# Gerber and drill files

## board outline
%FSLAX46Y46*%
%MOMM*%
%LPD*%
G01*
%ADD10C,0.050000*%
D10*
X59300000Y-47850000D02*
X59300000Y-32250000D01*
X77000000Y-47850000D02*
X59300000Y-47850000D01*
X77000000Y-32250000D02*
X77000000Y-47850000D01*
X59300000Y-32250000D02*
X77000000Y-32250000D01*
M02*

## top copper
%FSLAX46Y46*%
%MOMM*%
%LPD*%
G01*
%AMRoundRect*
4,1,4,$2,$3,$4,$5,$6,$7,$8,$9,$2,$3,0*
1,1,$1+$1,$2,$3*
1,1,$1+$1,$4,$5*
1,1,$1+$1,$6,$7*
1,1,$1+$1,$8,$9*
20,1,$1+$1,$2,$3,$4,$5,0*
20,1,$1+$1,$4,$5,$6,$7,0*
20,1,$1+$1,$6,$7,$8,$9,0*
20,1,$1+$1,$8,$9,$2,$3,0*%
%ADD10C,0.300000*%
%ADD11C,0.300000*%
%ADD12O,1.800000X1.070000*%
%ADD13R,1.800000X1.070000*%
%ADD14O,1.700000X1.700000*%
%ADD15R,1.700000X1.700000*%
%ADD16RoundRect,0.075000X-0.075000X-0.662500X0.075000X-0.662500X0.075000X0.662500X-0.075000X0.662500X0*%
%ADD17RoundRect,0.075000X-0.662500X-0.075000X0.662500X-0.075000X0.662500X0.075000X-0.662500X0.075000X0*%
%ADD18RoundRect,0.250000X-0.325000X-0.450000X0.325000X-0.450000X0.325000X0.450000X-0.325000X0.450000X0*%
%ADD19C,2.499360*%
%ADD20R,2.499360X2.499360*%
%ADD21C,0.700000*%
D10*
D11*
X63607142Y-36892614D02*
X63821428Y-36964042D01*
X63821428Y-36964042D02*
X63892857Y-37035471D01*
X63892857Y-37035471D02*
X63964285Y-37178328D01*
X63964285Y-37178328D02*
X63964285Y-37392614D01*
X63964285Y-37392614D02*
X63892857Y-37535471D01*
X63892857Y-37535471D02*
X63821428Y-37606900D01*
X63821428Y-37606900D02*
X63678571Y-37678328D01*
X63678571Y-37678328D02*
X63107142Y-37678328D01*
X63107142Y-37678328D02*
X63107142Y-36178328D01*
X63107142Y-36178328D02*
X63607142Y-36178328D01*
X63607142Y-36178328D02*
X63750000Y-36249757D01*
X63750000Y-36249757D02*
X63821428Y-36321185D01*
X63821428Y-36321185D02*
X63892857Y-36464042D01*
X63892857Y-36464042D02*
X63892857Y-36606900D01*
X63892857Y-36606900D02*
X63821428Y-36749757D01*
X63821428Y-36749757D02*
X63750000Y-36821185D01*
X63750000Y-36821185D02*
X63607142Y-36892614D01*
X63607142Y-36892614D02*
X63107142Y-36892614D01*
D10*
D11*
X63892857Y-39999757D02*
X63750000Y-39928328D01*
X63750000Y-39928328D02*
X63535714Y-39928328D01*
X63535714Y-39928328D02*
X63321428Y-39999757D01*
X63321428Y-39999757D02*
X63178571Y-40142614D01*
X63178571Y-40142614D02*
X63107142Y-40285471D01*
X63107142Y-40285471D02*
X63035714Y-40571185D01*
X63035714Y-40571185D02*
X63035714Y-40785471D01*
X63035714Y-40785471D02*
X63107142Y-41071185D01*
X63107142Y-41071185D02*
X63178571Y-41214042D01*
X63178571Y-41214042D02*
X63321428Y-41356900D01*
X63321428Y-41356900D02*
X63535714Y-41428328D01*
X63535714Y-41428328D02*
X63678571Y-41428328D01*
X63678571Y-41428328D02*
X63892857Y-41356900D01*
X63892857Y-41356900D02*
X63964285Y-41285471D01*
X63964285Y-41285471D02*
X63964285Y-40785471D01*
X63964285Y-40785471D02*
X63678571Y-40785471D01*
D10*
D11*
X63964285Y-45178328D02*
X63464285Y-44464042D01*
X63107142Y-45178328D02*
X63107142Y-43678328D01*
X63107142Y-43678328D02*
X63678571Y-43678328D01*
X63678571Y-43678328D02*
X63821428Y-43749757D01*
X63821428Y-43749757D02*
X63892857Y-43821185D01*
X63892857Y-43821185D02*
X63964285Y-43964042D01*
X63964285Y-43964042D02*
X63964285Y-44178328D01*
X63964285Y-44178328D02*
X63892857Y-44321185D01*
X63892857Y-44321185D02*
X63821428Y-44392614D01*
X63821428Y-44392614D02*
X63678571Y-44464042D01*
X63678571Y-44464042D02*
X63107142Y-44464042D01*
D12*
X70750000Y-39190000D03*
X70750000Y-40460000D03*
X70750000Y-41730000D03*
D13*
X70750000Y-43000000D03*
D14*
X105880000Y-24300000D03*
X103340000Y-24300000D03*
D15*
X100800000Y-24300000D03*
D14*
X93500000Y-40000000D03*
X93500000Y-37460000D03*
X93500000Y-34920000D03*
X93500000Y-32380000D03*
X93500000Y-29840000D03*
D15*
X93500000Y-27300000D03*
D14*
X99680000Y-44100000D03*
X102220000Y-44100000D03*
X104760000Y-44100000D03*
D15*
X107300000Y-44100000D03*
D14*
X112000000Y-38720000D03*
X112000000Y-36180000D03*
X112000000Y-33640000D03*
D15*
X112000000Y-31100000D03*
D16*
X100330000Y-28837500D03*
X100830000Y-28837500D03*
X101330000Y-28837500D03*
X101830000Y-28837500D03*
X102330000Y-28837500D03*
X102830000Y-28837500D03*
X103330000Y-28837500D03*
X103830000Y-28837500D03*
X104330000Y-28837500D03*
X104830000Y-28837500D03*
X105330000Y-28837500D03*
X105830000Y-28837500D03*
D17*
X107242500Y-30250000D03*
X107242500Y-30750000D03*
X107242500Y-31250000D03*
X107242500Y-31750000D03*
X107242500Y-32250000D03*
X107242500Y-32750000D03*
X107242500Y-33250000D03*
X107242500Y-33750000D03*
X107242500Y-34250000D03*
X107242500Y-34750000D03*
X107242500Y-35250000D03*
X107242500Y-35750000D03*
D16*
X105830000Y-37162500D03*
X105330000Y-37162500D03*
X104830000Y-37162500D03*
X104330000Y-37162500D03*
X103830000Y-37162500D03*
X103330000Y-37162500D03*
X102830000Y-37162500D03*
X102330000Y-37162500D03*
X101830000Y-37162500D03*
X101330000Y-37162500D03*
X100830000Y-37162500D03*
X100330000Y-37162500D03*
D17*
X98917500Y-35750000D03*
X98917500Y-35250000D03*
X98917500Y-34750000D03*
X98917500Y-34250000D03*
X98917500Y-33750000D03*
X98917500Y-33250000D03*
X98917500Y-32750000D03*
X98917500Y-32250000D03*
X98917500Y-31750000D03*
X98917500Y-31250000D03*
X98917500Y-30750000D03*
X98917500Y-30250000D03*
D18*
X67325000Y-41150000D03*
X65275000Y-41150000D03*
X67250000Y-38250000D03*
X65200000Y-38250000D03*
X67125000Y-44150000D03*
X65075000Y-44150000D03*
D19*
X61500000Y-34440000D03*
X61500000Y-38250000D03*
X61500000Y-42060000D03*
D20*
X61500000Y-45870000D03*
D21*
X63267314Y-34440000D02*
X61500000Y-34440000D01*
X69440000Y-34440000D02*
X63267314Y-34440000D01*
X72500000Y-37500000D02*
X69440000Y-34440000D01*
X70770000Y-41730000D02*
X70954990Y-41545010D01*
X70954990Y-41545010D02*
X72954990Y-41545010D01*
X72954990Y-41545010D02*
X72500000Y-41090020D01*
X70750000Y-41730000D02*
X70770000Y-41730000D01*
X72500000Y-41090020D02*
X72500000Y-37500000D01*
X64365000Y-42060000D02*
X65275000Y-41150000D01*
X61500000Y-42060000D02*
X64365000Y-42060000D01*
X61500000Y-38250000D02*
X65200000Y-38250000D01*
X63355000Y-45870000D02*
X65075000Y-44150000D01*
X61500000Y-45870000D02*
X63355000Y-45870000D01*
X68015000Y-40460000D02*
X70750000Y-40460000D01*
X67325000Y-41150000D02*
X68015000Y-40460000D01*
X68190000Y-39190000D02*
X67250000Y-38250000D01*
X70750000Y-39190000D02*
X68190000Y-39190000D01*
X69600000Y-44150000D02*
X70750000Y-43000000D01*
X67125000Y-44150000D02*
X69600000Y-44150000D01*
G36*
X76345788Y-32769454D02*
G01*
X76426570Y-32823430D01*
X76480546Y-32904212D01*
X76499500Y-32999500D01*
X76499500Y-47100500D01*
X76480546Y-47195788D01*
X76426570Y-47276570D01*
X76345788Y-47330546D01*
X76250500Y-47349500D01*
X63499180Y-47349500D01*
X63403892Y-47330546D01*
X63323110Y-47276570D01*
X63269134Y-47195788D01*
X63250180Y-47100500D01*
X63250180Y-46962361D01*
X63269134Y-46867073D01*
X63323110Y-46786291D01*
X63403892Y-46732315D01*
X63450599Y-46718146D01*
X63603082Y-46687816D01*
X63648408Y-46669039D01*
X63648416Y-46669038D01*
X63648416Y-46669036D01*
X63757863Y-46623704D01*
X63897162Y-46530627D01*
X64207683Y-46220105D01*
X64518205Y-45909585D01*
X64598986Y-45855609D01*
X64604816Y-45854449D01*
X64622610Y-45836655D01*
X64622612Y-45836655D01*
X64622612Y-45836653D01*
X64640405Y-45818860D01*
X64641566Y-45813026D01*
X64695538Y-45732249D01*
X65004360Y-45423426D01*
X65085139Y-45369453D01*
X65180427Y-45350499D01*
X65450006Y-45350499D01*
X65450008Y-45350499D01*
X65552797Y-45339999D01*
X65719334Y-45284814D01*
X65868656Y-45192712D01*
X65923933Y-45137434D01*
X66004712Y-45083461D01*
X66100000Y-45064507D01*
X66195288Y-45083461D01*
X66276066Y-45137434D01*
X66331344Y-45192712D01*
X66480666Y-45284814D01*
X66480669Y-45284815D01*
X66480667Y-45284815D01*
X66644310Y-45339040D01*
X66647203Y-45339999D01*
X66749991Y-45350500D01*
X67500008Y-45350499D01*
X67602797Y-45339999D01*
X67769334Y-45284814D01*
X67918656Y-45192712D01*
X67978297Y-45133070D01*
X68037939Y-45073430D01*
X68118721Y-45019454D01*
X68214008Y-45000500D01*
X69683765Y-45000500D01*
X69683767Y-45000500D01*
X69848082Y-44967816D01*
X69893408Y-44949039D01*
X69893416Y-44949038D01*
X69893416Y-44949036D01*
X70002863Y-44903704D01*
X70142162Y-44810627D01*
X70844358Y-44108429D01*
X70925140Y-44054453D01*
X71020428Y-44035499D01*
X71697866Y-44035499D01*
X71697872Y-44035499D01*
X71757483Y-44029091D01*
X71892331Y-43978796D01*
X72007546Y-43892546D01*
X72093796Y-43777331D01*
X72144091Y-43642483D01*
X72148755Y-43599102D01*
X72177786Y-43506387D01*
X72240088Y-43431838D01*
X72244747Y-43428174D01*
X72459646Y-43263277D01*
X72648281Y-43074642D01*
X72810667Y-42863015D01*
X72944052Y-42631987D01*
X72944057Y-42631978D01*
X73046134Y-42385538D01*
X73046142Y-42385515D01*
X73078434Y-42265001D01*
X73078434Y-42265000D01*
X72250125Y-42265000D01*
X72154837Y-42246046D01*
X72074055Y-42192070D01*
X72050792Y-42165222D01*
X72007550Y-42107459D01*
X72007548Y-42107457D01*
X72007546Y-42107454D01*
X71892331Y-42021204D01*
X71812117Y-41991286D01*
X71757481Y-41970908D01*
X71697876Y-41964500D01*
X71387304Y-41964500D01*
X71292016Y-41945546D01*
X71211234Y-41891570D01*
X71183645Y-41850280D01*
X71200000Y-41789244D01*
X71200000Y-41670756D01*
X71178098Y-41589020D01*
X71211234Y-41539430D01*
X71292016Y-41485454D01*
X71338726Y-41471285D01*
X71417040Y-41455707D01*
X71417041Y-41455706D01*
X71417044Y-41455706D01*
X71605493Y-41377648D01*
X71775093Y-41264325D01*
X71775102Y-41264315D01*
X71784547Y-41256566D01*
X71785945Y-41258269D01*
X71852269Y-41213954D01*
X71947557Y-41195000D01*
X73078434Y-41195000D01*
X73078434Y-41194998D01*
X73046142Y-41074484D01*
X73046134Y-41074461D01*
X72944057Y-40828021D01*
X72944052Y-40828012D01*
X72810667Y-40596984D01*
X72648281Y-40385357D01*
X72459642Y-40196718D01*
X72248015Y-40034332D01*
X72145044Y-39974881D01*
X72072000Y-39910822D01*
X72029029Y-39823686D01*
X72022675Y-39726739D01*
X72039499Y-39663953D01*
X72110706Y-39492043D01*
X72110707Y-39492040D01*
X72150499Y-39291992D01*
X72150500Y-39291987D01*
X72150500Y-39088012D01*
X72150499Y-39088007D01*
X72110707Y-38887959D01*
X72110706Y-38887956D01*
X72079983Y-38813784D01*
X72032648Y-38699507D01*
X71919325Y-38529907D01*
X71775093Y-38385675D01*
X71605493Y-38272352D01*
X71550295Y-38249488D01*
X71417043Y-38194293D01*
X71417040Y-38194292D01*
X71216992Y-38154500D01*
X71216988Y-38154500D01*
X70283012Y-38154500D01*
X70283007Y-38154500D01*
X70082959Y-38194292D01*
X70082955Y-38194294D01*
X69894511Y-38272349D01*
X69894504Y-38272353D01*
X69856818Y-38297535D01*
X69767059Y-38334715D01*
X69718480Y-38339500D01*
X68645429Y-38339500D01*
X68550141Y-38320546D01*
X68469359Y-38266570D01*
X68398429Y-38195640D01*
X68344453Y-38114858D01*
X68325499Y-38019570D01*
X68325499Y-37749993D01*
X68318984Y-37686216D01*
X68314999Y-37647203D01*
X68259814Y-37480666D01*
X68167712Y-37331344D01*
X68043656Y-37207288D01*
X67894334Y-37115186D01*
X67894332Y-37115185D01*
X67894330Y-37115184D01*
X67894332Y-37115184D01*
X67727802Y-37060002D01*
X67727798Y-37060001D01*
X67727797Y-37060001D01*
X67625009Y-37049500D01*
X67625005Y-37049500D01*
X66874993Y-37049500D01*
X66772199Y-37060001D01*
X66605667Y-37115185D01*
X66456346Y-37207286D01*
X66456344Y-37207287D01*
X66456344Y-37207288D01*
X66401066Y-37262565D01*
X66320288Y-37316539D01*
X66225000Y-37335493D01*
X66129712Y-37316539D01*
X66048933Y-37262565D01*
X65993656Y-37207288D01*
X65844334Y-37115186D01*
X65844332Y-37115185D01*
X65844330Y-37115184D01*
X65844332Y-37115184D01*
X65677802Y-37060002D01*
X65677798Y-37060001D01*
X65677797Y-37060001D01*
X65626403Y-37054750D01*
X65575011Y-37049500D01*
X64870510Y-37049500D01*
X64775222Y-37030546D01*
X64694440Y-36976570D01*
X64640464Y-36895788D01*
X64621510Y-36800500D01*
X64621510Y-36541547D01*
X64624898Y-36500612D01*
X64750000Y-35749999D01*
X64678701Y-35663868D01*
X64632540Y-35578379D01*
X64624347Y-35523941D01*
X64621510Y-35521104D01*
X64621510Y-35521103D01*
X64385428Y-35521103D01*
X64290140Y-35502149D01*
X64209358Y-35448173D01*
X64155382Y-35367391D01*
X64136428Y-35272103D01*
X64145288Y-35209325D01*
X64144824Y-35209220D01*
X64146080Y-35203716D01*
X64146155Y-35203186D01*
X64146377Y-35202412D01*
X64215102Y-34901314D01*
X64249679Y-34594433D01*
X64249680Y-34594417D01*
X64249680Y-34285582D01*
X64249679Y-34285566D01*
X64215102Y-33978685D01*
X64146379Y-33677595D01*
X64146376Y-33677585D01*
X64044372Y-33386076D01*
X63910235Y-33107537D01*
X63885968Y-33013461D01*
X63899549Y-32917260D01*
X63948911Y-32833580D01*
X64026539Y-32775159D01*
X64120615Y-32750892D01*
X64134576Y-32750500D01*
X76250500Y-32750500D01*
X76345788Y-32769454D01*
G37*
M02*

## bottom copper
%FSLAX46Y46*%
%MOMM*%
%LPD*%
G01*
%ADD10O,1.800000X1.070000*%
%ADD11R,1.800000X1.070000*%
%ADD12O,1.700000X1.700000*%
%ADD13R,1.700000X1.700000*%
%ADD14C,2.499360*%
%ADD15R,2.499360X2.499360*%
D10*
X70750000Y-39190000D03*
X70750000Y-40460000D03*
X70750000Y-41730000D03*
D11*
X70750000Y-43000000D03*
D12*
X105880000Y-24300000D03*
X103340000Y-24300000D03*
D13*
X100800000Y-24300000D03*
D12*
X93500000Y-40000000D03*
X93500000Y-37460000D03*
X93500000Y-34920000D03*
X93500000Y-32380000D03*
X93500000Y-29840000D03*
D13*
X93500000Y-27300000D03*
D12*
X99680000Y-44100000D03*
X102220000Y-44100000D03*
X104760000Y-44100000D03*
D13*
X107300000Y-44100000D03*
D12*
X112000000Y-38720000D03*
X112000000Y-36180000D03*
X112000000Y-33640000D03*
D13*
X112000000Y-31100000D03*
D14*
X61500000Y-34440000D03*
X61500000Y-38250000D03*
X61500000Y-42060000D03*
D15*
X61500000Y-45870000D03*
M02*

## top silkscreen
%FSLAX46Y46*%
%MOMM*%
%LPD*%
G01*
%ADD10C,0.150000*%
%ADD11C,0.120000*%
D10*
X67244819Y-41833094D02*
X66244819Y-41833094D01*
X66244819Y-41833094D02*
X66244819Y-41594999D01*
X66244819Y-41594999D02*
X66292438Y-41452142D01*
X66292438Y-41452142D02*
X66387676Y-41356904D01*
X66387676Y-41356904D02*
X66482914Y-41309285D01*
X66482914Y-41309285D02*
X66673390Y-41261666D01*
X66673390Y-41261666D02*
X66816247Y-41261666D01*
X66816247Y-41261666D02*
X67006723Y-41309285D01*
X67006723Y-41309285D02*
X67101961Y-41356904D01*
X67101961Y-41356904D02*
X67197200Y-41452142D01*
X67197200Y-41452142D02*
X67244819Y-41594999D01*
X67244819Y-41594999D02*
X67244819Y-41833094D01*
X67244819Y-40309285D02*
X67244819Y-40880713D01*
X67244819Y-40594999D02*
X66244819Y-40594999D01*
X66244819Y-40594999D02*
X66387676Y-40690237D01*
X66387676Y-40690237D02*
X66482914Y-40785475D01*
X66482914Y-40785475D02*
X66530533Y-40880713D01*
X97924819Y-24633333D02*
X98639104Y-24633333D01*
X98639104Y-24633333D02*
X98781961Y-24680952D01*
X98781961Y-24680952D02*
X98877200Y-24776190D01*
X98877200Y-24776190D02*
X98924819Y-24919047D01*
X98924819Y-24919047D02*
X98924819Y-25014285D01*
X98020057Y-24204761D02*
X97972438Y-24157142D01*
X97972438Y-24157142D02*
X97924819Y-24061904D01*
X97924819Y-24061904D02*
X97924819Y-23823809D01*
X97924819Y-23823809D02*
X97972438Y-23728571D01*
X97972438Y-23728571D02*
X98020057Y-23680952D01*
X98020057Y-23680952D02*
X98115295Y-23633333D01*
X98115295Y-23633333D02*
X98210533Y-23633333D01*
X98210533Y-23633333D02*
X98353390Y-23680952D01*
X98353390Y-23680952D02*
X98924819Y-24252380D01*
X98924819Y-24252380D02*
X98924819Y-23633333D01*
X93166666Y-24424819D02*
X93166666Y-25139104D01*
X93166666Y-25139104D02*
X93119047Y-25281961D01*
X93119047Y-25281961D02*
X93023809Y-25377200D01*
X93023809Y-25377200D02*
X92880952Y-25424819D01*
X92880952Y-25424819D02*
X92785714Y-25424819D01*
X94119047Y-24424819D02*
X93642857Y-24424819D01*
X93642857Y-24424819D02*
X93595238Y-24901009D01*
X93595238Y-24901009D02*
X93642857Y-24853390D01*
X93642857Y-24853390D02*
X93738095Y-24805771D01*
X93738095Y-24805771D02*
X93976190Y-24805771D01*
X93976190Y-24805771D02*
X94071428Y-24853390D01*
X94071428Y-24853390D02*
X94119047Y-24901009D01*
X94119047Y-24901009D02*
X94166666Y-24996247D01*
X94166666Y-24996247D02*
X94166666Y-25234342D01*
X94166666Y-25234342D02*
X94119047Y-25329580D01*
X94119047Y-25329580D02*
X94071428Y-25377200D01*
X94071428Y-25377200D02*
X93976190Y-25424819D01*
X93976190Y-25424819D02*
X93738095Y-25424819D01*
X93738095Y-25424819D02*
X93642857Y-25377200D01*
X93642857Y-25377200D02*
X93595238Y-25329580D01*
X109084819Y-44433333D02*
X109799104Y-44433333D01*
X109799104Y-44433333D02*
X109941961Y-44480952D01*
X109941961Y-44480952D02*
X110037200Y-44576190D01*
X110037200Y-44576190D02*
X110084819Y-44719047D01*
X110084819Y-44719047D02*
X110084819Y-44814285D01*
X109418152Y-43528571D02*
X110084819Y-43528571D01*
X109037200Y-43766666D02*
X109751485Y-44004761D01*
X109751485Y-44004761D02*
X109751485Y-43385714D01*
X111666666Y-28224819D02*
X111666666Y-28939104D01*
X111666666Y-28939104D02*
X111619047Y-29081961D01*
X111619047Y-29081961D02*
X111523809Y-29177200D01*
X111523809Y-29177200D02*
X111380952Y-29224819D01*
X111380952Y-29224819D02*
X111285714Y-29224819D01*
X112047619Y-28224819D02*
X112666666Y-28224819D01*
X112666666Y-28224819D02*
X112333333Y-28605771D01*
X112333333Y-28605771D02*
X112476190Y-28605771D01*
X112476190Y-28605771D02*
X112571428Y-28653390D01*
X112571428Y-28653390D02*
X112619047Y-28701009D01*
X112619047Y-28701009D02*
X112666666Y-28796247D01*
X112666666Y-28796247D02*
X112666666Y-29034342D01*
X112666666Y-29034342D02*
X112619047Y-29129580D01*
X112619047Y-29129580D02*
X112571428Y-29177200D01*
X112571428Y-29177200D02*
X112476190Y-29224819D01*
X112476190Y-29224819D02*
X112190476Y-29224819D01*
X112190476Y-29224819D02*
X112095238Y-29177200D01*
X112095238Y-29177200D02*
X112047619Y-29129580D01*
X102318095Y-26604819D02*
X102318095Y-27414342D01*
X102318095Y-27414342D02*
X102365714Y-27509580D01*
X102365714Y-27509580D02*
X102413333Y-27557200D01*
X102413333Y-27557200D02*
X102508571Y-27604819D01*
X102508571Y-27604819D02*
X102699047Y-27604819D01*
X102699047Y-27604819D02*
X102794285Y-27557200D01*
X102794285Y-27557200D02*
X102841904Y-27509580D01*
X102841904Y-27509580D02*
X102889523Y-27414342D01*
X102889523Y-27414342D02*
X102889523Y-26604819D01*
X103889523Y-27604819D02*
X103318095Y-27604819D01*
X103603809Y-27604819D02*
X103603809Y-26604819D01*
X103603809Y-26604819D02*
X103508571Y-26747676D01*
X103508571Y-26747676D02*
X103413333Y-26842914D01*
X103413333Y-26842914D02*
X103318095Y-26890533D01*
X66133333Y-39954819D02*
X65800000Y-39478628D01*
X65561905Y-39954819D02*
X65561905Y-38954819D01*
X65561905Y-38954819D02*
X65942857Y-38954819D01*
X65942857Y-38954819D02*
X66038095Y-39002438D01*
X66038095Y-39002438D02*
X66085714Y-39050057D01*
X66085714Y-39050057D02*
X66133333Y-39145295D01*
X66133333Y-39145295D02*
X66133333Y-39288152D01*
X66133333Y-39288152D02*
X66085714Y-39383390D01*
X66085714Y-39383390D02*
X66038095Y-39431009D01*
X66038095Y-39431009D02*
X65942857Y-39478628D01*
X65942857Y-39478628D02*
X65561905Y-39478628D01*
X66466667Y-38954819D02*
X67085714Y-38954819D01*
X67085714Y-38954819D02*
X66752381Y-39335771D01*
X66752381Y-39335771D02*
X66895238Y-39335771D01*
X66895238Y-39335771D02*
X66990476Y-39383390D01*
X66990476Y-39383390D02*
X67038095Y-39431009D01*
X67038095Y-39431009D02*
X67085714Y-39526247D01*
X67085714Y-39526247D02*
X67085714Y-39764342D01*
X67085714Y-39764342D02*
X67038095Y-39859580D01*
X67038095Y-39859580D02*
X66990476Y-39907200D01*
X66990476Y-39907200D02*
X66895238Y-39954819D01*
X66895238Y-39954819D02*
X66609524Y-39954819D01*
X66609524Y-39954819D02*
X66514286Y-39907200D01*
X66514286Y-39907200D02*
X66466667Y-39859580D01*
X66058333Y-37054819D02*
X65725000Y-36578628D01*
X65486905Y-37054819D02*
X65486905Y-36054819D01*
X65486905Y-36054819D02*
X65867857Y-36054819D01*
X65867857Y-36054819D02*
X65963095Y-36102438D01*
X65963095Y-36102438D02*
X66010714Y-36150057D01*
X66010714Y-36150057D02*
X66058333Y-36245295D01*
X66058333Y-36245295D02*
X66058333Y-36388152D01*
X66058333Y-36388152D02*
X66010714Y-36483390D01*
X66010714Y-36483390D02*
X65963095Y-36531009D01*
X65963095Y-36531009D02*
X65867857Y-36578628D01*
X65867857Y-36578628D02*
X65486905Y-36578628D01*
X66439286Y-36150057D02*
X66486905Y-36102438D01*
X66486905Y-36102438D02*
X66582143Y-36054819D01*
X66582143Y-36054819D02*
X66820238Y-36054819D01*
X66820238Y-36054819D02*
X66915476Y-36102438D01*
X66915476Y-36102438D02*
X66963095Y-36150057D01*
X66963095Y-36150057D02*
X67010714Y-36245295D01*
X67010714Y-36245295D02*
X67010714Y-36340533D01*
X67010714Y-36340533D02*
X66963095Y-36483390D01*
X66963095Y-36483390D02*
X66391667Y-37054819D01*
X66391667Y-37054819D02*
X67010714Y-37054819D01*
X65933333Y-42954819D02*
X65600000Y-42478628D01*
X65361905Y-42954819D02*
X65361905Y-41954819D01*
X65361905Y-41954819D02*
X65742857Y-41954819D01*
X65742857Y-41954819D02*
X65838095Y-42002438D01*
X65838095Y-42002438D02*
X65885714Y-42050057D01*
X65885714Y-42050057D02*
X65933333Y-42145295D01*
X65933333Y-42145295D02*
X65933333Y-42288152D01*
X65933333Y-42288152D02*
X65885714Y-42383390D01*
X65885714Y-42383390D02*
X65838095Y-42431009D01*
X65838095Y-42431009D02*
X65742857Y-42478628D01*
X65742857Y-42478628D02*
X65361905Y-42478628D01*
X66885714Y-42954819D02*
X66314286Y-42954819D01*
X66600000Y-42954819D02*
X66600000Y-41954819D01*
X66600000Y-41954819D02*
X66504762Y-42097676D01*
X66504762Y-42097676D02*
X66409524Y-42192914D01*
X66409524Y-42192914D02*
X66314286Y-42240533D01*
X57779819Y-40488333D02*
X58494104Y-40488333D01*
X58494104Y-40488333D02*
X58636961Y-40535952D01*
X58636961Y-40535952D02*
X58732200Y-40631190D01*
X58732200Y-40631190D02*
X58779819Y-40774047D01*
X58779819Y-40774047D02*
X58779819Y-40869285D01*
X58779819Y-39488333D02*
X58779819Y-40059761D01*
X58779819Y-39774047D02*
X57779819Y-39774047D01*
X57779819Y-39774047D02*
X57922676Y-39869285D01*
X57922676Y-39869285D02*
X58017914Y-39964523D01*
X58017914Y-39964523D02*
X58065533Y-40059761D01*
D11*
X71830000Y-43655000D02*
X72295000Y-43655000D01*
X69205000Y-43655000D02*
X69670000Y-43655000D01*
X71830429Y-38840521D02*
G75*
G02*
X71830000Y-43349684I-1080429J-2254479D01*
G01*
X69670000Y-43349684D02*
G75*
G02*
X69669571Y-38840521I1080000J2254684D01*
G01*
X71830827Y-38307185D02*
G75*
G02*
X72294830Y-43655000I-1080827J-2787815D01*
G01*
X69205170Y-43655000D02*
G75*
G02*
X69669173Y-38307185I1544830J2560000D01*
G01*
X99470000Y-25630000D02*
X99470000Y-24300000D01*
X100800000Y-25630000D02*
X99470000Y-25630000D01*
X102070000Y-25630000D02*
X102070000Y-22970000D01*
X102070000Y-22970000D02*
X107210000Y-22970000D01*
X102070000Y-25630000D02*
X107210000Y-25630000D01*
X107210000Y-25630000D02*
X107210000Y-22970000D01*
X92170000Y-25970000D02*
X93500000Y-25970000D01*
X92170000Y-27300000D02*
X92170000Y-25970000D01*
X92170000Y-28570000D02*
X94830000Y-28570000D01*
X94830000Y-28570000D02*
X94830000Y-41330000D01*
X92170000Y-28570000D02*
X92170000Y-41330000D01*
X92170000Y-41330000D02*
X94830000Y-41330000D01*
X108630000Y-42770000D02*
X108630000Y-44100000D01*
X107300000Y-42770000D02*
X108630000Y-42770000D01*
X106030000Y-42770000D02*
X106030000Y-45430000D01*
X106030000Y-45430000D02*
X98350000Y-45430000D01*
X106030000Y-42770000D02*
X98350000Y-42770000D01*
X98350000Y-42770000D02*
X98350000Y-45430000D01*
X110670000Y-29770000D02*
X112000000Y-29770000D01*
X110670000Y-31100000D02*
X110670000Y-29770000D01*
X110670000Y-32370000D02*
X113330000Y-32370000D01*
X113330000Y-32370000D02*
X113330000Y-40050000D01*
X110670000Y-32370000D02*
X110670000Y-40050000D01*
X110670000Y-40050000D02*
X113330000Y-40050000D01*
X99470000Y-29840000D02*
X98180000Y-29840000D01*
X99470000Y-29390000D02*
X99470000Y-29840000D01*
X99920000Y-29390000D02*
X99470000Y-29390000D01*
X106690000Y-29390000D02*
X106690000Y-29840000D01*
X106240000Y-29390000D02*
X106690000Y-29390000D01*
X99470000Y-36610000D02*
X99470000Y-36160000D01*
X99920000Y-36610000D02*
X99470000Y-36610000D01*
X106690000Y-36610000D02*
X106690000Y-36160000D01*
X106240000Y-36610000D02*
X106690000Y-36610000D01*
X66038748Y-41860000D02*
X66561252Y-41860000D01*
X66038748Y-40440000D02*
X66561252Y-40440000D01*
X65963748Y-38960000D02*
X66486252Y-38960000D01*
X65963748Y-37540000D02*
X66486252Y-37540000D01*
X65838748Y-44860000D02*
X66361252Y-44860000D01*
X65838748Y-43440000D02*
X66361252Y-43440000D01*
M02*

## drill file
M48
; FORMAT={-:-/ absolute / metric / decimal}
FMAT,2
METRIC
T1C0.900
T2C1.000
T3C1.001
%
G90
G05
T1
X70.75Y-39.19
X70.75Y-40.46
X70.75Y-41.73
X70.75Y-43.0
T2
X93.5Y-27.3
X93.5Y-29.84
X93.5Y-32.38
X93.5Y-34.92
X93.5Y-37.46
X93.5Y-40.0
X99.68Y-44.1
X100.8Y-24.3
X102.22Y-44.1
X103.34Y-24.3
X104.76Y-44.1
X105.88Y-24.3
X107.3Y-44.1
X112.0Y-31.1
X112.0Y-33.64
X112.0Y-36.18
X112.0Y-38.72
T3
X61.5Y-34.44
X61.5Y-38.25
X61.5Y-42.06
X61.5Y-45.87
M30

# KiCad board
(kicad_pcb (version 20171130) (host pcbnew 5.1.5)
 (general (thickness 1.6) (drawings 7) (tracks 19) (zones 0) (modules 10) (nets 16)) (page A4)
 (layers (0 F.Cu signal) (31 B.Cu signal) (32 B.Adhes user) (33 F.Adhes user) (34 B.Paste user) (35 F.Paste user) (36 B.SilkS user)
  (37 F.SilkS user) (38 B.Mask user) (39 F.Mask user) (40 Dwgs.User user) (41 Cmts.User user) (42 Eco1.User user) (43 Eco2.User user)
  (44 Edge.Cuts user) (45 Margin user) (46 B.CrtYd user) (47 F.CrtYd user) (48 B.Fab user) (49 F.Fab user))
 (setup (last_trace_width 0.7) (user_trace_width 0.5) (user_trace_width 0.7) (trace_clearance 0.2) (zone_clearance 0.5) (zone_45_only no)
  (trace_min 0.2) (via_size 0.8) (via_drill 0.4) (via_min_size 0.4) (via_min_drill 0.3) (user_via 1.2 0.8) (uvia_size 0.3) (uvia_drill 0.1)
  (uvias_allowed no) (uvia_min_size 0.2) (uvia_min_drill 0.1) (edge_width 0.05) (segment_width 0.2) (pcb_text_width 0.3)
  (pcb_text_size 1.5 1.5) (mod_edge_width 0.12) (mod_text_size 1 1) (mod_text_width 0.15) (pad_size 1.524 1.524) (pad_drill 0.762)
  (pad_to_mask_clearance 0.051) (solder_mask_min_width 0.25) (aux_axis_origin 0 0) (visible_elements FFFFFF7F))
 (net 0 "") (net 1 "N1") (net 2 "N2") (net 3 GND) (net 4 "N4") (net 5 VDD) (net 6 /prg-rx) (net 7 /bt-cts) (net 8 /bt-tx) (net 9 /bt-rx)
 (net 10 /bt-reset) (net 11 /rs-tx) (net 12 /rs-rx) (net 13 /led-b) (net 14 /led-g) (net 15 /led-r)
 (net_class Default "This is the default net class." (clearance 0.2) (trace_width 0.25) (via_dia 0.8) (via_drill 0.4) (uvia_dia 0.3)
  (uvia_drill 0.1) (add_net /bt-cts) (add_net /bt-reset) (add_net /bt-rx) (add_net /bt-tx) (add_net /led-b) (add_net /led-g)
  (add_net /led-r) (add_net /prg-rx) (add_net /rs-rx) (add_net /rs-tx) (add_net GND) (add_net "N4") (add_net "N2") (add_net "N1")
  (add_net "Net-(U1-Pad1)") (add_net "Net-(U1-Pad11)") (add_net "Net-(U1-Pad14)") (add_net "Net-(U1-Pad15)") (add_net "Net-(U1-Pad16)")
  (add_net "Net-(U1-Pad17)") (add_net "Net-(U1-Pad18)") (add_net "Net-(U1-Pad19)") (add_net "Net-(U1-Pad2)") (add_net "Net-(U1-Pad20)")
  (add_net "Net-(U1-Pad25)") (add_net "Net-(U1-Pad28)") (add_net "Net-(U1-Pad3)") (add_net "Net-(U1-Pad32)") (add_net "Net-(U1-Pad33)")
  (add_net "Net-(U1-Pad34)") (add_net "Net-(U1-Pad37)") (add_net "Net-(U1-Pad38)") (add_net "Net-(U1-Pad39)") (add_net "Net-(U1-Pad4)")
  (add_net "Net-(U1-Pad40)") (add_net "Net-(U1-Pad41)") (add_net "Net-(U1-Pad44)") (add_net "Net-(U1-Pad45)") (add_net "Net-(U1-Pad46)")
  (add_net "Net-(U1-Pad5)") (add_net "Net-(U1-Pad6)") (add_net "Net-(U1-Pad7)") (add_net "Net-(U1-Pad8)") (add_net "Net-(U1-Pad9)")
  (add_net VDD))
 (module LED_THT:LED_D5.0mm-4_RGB (layer F.Cu) (at 70.75 43 90)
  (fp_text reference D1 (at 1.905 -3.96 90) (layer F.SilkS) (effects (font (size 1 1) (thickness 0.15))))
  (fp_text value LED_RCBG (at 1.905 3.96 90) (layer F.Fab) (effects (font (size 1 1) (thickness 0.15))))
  (fp_line (start -0.655 1.08) (end -0.655 1.545) (layer F.SilkS) (width 0.12))
  (fp_line (start -0.655 -1.545) (end -0.655 -1.08) (layer F.SilkS) (width 0.12))
  (fp_arc (start 1.905 0) (end -0.349684 1.08) (angle -128.8) (layer F.SilkS) (width 0.12))
  (fp_arc (start 1.905 0) (end -0.349684 -1.08) (angle 128.8) (layer F.SilkS) (width 0.12))
  (fp_arc (start 1.905 0) (end -0.655 1.54483) (angle -127.7) (layer F.SilkS) (width 0.12))
  (fp_arc (start 1.905 0) (end -0.655 -1.54483) (angle 127.7) (layer F.SilkS) (width 0.12))
  (pad 4 thru_hole oval (at 3.81 0 90) (size 1.07 1.8) (drill 0.9) (layers *.Cu *.Mask) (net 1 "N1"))
  (pad 3 thru_hole oval (at 2.54 0 90) (size 1.07 1.8) (drill 0.9) (layers *.Cu *.Mask) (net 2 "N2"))
  (pad 2 thru_hole oval (at 1.27 0 90) (size 1.07 1.8) (drill 0.9) (layers *.Cu *.Mask) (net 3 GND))
  (pad 1 thru_hole rect (at 0 0 90) (size 1.07 1.8) (drill 0.9) (layers *.Cu *.Mask) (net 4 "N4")))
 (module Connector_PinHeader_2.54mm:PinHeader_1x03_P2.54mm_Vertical (layer F.Cu) (at 100.8 24.3 90)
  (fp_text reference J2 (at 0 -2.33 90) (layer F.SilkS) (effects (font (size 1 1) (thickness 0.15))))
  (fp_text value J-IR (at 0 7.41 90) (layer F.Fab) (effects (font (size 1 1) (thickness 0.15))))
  (fp_line (start -1.33 -1.33) (end 0 -1.33) (layer F.SilkS) (width 0.12))
  (fp_line (start -1.33 0) (end -1.33 -1.33) (layer F.SilkS) (width 0.12))
  (fp_line (start -1.33 1.27) (end 1.33 1.27) (layer F.SilkS) (width 0.12))
  (fp_line (start 1.33 1.27) (end 1.33 6.41) (layer F.SilkS) (width 0.12))
  (fp_line (start -1.33 1.27) (end -1.33 6.41) (layer F.SilkS) (width 0.12))
  (fp_line (start -1.33 6.41) (end 1.33 6.41) (layer F.SilkS) (width 0.12))
  (pad 3 thru_hole oval (at 0 5.08 90) (size 1.7 1.7) (drill 1) (layers *.Cu *.Mask) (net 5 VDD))
  (pad 2 thru_hole oval (at 0 2.54 90) (size 1.7 1.7) (drill 1) (layers *.Cu *.Mask) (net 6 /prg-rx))
  (pad 1 thru_hole rect (at 0 0 90) (size 1.7 1.7) (drill 1) (layers *.Cu *.Mask) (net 3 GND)))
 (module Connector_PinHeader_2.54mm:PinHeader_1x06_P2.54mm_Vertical (layer F.Cu) (at 93.5 27.3)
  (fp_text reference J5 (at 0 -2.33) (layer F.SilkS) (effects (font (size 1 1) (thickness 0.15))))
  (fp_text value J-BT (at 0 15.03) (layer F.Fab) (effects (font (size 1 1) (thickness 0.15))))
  (fp_line (start -1.33 -1.33) (end 0 -1.33) (layer F.SilkS) (width 0.12))
  (fp_line (start -1.33 0) (end -1.33 -1.33) (layer F.SilkS) (width 0.12))
  (fp_line (start -1.33 1.27) (end 1.33 1.27) (layer F.SilkS) (width 0.12))
  (fp_line (start 1.33 1.27) (end 1.33 14.03) (layer F.SilkS) (width 0.12))
  (fp_line (start -1.33 1.27) (end -1.33 14.03) (layer F.SilkS) (width 0.12))
  (fp_line (start -1.33 14.03) (end 1.33 14.03) (layer F.SilkS) (width 0.12))
  (pad 6 thru_hole oval (at 0 12.7) (size 1.7 1.7) (drill 1) (layers *.Cu *.Mask) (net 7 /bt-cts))
  (pad 5 thru_hole oval (at 0 10.16) (size 1.7 1.7) (drill 1) (layers *.Cu *.Mask) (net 5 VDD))
  (pad 4 thru_hole oval (at 0 7.62) (size 1.7 1.7) (drill 1) (layers *.Cu *.Mask) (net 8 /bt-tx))
  (pad 3 thru_hole oval (at 0 5.08) (size 1.7 1.7) (drill 1) (layers *.Cu *.Mask) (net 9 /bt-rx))
  (pad 2 thru_hole oval (at 0 2.54) (size 1.7 1.7) (drill 1) (layers *.Cu *.Mask) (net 3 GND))
  (pad 1 thru_hole rect (at 0 0) (size 1.7 1.7) (drill 1) (layers *.Cu *.Mask) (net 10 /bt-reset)))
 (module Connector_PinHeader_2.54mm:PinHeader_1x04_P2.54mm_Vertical (layer F.Cu) (at 107.3 44.1 270)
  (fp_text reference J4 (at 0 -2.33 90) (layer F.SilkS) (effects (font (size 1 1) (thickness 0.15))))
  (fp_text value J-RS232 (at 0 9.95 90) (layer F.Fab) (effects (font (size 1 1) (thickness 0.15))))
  (fp_line (start -1.33 -1.33) (end 0 -1.33) (layer F.SilkS) (width 0.12))
  (fp_line (start -1.33 0) (end -1.33 -1.33) (layer F.SilkS) (width 0.12))
  (fp_line (start -1.33 1.27) (end 1.33 1.27) (layer F.SilkS) (width 0.12))
  (fp_line (start 1.33 1.27) (end 1.33 8.95) (layer F.SilkS) (width 0.12))
  (fp_line (start -1.33 1.27) (end -1.33 8.95) (layer F.SilkS) (width 0.12))
  (fp_line (start -1.33 8.95) (end 1.33 8.95) (layer F.SilkS) (width 0.12))
  (pad 4 thru_hole oval (at 0 7.62 270) (size 1.7 1.7) (drill 1) (layers *.Cu *.Mask) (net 5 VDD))
  (pad 3 thru_hole oval (at 0 5.08 270) (size 1.7 1.7) (drill 1) (layers *.Cu *.Mask) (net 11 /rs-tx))
  (pad 2 thru_hole oval (at 0 2.54 270) (size 1.7 1.7) (drill 1) (layers *.Cu *.Mask) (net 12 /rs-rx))
  (pad 1 thru_hole rect (at 0 0 270) (size 1.7 1.7) (drill 1) (layers *.Cu *.Mask) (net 3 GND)))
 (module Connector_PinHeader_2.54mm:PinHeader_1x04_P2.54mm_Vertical (layer F.Cu) (at 112 31.1)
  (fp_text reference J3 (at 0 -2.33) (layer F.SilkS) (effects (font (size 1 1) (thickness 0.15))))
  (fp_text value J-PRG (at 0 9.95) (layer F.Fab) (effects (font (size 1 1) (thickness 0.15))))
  (fp_line (start -1.33 -1.33) (end 0 -1.33) (layer F.SilkS) (width 0.12))
  (fp_line (start -1.33 0) (end -1.33 -1.33) (layer F.SilkS) (width 0.12))
  (fp_line (start -1.33 1.27) (end 1.33 1.27) (layer F.SilkS) (width 0.12))
  (fp_line (start 1.33 1.27) (end 1.33 8.95) (layer F.SilkS) (width 0.12))
  (fp_line (start -1.33 1.27) (end -1.33 8.95) (layer F.SilkS) (width 0.12))
  (fp_line (start -1.33 8.95) (end 1.33 8.95) (layer F.SilkS) (width 0.12))
  (pad 4 thru_hole oval (at 0 7.62) (size 1.7 1.7) (drill 1) (layers *.Cu *.Mask) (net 5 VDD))
  (pad 3 thru_hole oval (at 0 5.08) (size 1.7 1.7) (drill 1) (layers *.Cu *.Mask) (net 7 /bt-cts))
  (pad 2 thru_hole oval (at 0 2.54) (size 1.7 1.7) (drill 1) (layers *.Cu *.Mask) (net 6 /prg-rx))
  (pad 1 thru_hole rect (at 0 0) (size 1.7 1.7) (drill 1) (layers *.Cu *.Mask) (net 3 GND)))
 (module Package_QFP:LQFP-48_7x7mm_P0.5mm (layer F.Cu) (at 103.08 33)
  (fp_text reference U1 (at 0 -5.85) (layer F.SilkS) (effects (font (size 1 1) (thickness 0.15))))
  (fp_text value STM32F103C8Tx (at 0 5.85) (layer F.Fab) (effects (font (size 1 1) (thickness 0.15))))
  (fp_line (start -3.61 -3.16) (end -4.9 -3.16) (layer F.SilkS) (width 0.12))
  (fp_line (start -3.61 -3.61) (end -3.61 -3.16) (layer F.SilkS) (width 0.12))
  (fp_line (start -3.16 -3.61) (end -3.61 -3.61) (layer F.SilkS) (width 0.12))
  (fp_line (start 3.61 -3.61) (end 3.61 -3.16) (layer F.SilkS) (width 0.12))
  (fp_line (start 3.16 -3.61) (end 3.61 -3.61) (layer F.SilkS) (width 0.12))
  (fp_line (start -3.61 3.61) (end -3.61 3.16) (layer F.SilkS) (width 0.12))
  (fp_line (start -3.16 3.61) (end -3.61 3.61) (layer F.SilkS) (width 0.12))
  (fp_line (start 3.61 3.61) (end 3.61 3.16) (layer F.SilkS) (width 0.12))
  (fp_line (start 3.16 3.61) (end 3.61 3.61) (layer F.SilkS) (width 0.12))
  (pad 48 smd roundrect (at -2.75 -4.1625) (size 0.3 1.475) (layers F.Cu F.Paste F.Mask) (roundrect_rratio 0.25) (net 5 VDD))
  (pad 47 smd roundrect (at -2.25 -4.1625) (size 0.3 1.475) (layers F.Cu F.Paste F.Mask) (roundrect_rratio 0.25) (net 3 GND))
  (pad 46 smd roundrect (at -1.75 -4.1625) (size 0.3 1.475) (layers F.Cu F.Paste F.Mask) (roundrect_rratio 0.25))
  (pad 45 smd roundrect (at -1.25 -4.1625) (size 0.3 1.475) (layers F.Cu F.Paste F.Mask) (roundrect_rratio 0.25))
  (pad 44 smd roundrect (at -0.75 -4.1625) (size 0.3 1.475) (layers F.Cu F.Paste F.Mask) (roundrect_rratio 0.25))
  (pad 43 smd roundrect (at -0.25 -4.1625) (size 0.3 1.475) (layers F.Cu F.Paste F.Mask) (roundrect_rratio 0.25) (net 6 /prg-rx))
  (pad 42 smd roundrect (at 0.25 -4.1625) (size 0.3 1.475) (layers F.Cu F.Paste F.Mask) (roundrect_rratio 0.25) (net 7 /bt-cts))
  (pad 41 smd roundrect (at 0.75 -4.1625) (size 0.3 1.475) (layers F.Cu F.Paste F.Mask) (roundrect_rratio 0.25))
  (pad 40 smd roundrect (at 1.25 -4.1625) (size 0.3 1.475) (layers F.Cu F.Paste F.Mask) (roundrect_rratio 0.25))
  (pad 39 smd roundrect (at 1.75 -4.1625) (size 0.3 1.475) (layers F.Cu F.Paste F.Mask) (roundrect_rratio 0.25))
  (pad 38 smd roundrect (at 2.25 -4.1625) (size 0.3 1.475) (layers F.Cu F.Paste F.Mask) (roundrect_rratio 0.25))
  (pad 37 smd roundrect (at 2.75 -4.1625) (size 0.3 1.475) (layers F.Cu F.Paste F.Mask) (roundrect_rratio 0.25))
  (pad 36 smd roundrect (at 4.1625 -2.75) (size 1.475 0.3) (layers F.Cu F.Paste F.Mask) (roundrect_rratio 0.25) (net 5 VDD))
  (pad 35 smd roundrect (at 4.1625 -2.25) (size 1.475 0.3) (layers F.Cu F.Paste F.Mask) (roundrect_rratio 0.25) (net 3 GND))
  (pad 34 smd roundrect (at 4.1625 -1.75) (size 1.475 0.3) (layers F.Cu F.Paste F.Mask) (roundrect_rratio 0.25))
  (pad 33 smd roundrect (at 4.1625 -1.25) (size 1.475 0.3) (layers F.Cu F.Paste F.Mask) (roundrect_rratio 0.25))
  (pad 32 smd roundrect (at 4.1625 -0.75) (size 1.475 0.3) (layers F.Cu F.Paste F.Mask) (roundrect_rratio 0.25))
  (pad 31 smd roundrect (at 4.1625 -0.25) (size 1.475 0.3) (layers F.Cu F.Paste F.Mask) (roundrect_rratio 0.25) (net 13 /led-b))
  (pad 30 smd roundrect (at 4.1625 0.25) (size 1.475 0.3) (layers F.Cu F.Paste F.Mask) (roundrect_rratio 0.25) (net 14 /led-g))
  (pad 29 smd roundrect (at 4.1625 0.75) (size 1.475 0.3) (layers F.Cu F.Paste F.Mask) (roundrect_rratio 0.25) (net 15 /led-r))
  (pad 28 smd roundrect (at 4.1625 1.25) (size 1.475 0.3) (layers F.Cu F.Paste F.Mask) (roundrect_rratio 0.25))
  (pad 27 smd roundrect (at 4.1625 1.75) (size 1.475 0.3) (layers F.Cu F.Paste F.Mask) (roundrect_rratio 0.25) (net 10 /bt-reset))
  (pad 26 smd roundrect (at 4.1625 2.25) (size 1.475 0.3) (layers F.Cu F.Paste F.Mask) (roundrect_rratio 0.25) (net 7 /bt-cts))
  (pad 25 smd roundrect (at 4.1625 2.75) (size 1.475 0.3) (layers F.Cu F.Paste F.Mask) (roundrect_rratio 0.25))
  (pad 24 smd roundrect (at 2.75 4.1625) (size 0.3 1.475) (layers F.Cu F.Paste F.Mask) (roundrect_rratio 0.25) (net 5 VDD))
  (pad 23 smd roundrect (at 2.25 4.1625) (size 0.3 1.475) (layers F.Cu F.Paste F.Mask) (roundrect_rratio 0.25) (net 3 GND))
  (pad 22 smd roundrect (at 1.75 4.1625) (size 0.3 1.475) (layers F.Cu F.Paste F.Mask) (roundrect_rratio 0.25) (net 12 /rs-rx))
  (pad 21 smd roundrect (at 1.25 4.1625) (size 0.3 1.475) (layers F.Cu F.Paste F.Mask) (roundrect_rratio 0.25) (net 11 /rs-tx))
  (pad 20 smd roundrect (at 0.75 4.1625) (size 0.3 1.475) (layers F.Cu F.Paste F.Mask) (roundrect_rratio 0.25))
  (pad 19 smd roundrect (at 0.25 4.1625) (size 0.3 1.475) (layers F.Cu F.Paste F.Mask) (roundrect_rratio 0.25))
  (pad 18 smd roundrect (at -0.25 4.1625) (size 0.3 1.475) (layers F.Cu F.Paste F.Mask) (roundrect_rratio 0.25))
  (pad 17 smd roundrect (at -0.75 4.1625) (size 0.3 1.475) (layers F.Cu F.Paste F.Mask) (roundrect_rratio 0.25))
  (pad 16 smd roundrect (at -1.25 4.1625) (size 0.3 1.475) (layers F.Cu F.Paste F.Mask) (roundrect_rratio 0.25))
  (pad 15 smd roundrect (at -1.75 4.1625) (size 0.3 1.475) (layers F.Cu F.Paste F.Mask) (roundrect_rratio 0.25))
  (pad 14 smd roundrect (at -2.25 4.1625) (size 0.3 1.475) (layers F.Cu F.Paste F.Mask) (roundrect_rratio 0.25))
  (pad 13 smd roundrect (at -2.75 4.1625) (size 0.3 1.475) (layers F.Cu F.Paste F.Mask) (roundrect_rratio 0.25) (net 9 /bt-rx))
  (pad 12 smd roundrect (at -4.1625 2.75) (size 1.475 0.3) (layers F.Cu F.Paste F.Mask) (roundrect_rratio 0.25) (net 8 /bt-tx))
  (pad 11 smd roundrect (at -4.1625 2.25) (size 1.475 0.3) (layers F.Cu F.Paste F.Mask) (roundrect_rratio 0.25))
  (pad 10 smd roundrect (at -4.1625 1.75) (size 1.475 0.3) (layers F.Cu F.Paste F.Mask) (roundrect_rratio 0.25) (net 7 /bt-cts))
  (pad 9 smd roundrect (at -4.1625 1.25) (size 1.475 0.3) (layers F.Cu F.Paste F.Mask) (roundrect_rratio 0.25))
  (pad 8 smd roundrect (at -4.1625 0.75) (size 1.475 0.3) (layers F.Cu F.Paste F.Mask) (roundrect_rratio 0.25))
  (pad 7 smd roundrect (at -4.1625 0.25) (size 1.475 0.3) (layers F.Cu F.Paste F.Mask) (roundrect_rratio 0.25))
  (pad 6 smd roundrect (at -4.1625 -0.25) (size 1.475 0.3) (layers F.Cu F.Paste F.Mask) (roundrect_rratio 0.25))
  (pad 5 smd roundrect (at -4.1625 -0.75) (size 1.475 0.3) (layers F.Cu F.Paste F.Mask) (roundrect_rratio 0.25))
  (pad 4 smd roundrect (at -4.1625 -1.25) (size 1.475 0.3) (layers F.Cu F.Paste F.Mask) (roundrect_rratio 0.25))
  (pad 3 smd roundrect (at -4.1625 -1.75) (size 1.475 0.3) (layers F.Cu F.Paste F.Mask) (roundrect_rratio 0.25))
  (pad 2 smd roundrect (at -4.1625 -2.25) (size 1.475 0.3) (layers F.Cu F.Paste F.Mask) (roundrect_rratio 0.25))
  (pad 1 smd roundrect (at -4.1625 -2.75) (size 1.475 0.3) (layers F.Cu F.Paste F.Mask) (roundrect_rratio 0.25)))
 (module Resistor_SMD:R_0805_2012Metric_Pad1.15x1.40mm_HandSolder (layer F.Cu) (at 66.3 41.15)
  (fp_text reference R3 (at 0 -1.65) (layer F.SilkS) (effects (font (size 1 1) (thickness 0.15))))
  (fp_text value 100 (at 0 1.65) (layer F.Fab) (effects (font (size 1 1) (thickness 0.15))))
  (fp_line (start -0.261252 0.71) (end 0.261252 0.71) (layer F.SilkS) (width 0.12))
  (fp_line (start -0.261252 -0.71) (end 0.261252 -0.71) (layer F.SilkS) (width 0.12))
  (pad 2 smd roundrect (at 1.025 0) (size 1.15 1.4) (layers F.Cu F.Paste F.Mask) (roundrect_rratio 0.217391) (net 2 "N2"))
  (pad 1 smd roundrect (at -1.025 0) (size 1.15 1.4) (layers F.Cu F.Paste F.Mask) (roundrect_rratio 0.217391) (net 13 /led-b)))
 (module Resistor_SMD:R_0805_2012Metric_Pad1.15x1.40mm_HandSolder (layer F.Cu) (at 66.225 38.25)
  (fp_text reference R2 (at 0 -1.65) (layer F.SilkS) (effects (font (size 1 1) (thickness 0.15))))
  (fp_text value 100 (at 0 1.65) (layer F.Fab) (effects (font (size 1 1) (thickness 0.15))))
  (fp_line (start -0.261252 0.71) (end 0.261252 0.71) (layer F.SilkS) (width 0.12))
  (fp_line (start -0.261252 -0.71) (end 0.261252 -0.71) (layer F.SilkS) (width 0.12))
  (pad 2 smd roundrect (at 1.025 0) (size 1.15 1.4) (layers F.Cu F.Paste F.Mask) (roundrect_rratio 0.217391) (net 1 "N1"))
  (pad 1 smd roundrect (at -1.025 0) (size 1.15 1.4) (layers F.Cu F.Paste F.Mask) (roundrect_rratio 0.217391) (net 14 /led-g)))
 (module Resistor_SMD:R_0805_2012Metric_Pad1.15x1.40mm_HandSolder (layer F.Cu) (at 66.1 44.15)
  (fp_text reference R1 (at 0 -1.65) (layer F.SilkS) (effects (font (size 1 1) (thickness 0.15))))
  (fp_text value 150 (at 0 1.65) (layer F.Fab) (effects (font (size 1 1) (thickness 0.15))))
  (fp_line (start -0.261252 0.71) (end 0.261252 0.71) (layer F.SilkS) (width 0.12))
  (fp_line (start -0.261252 -0.71) (end 0.261252 -0.71) (layer F.SilkS) (width 0.12))
  (pad 2 smd roundrect (at 1.025 0) (size 1.15 1.4) (layers F.Cu F.Paste F.Mask) (roundrect_rratio 0.217391) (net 4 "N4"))
  (pad 1 smd roundrect (at -1.025 0) (size 1.15 1.4) (layers F.Cu F.Paste F.Mask) (roundrect_rratio 0.217391) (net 15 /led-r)))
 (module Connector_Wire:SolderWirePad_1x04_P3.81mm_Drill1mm (layer F.Cu) (at 61.5 45.87 90)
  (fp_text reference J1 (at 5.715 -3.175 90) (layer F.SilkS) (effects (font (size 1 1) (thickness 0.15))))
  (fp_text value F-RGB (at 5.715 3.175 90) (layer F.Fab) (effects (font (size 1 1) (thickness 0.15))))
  (pad 4 thru_hole circle (at 11.43 0 90) (size 2.49936 2.49936) (drill 1.00076) (layers *.Cu *.Mask) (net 3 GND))
  (pad 3 thru_hole circle (at 7.62 0 90) (size 2.49936 2.49936) (drill 1.00076) (layers *.Cu *.Mask) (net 14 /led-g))
  (pad 2 thru_hole circle (at 3.81 0 90) (size 2.49936 2.49936) (drill 1.00076) (layers *.Cu *.Mask) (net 13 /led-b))
  (pad 1 thru_hole rect (at 0 0 90) (size 2.49936 2.49936) (drill 1.00076) (layers *.Cu *.Mask) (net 15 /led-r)))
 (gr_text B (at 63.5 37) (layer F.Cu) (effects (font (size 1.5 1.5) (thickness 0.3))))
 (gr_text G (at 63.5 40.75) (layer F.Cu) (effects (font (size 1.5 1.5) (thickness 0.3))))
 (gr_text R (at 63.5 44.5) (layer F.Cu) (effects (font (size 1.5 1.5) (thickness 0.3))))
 (gr_line (start 59.3 47.85) (end 59.3 32.25) (layer Edge.Cuts) (width 0.05))
 (gr_line (start 77 47.85) (end 59.3 47.85) (layer Edge.Cuts) (width 0.05))
 (gr_line (start 77 32.25) (end 77 47.85) (layer Edge.Cuts) (width 0.05))
 (gr_line (start 59.3 32.25) (end 77 32.25) (layer Edge.Cuts) (width 0.05))
 (segment (start 63.267314 34.44) (end 61.5 34.44) (width 0.7) (layer F.Cu) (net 3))
 (segment (start 69.44 34.44) (end 63.267314 34.44) (width 0.7) (layer F.Cu) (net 3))
 (segment (start 72.5 37.5) (end 69.44 34.44) (width 0.7) (layer F.Cu) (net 3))
 (segment (start 70.77 41.73) (end 70.95499 41.54501) (width 0.7) (layer F.Cu) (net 3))
 (segment (start 70.95499 41.54501) (end 72.95499 41.54501) (width 0.7) (layer F.Cu) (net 3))
 (segment (start 72.95499 41.54501) (end 72.5 41.09002) (width 0.7) (layer F.Cu) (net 3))
 (segment (start 70.75 41.73) (end 70.77 41.73) (width 0.7) (layer F.Cu) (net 3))
 (segment (start 72.5 41.09002) (end 72.5 37.5) (width 0.7) (layer F.Cu) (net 3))
 (segment (start 64.365 42.06) (end 65.275 41.15) (width 0.7) (layer F.Cu) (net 13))
 (segment (start 61.5 42.06) (end 64.365 42.06) (width 0.7) (layer F.Cu) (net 13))
 (segment (start 61.5 38.25) (end 65.2 38.25) (width 0.7) (layer F.Cu) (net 14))
 (segment (start 63.355 45.87) (end 65.075 44.15) (width 0.7) (layer F.Cu) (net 15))
 (segment (start 61.5 45.87) (end 63.355 45.87) (width 0.7) (layer F.Cu) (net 15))
 (segment (start 68.015 40.46) (end 70.75 40.46) (width 0.7) (layer F.Cu) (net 2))
 (segment (start 67.325 41.15) (end 68.015 40.46) (width 0.7) (layer F.Cu) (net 2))
 (segment (start 68.19 39.19) (end 67.25 38.25) (width 0.7) (layer F.Cu) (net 1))
 (segment (start 70.75 39.19) (end 68.19 39.19) (width 0.7) (layer F.Cu) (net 1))
 (segment (start 69.6 44.15) (end 70.75 43) (width 0.7) (layer F.Cu) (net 4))
 (segment (start 67.125 44.15) (end 69.6 44.15) (width 0.7) (layer F.Cu) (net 4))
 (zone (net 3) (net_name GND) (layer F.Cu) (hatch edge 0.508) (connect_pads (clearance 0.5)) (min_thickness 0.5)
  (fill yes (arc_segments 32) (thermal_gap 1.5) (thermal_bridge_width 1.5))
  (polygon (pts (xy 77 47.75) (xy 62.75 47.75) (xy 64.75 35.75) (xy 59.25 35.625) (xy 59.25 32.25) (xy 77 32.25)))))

